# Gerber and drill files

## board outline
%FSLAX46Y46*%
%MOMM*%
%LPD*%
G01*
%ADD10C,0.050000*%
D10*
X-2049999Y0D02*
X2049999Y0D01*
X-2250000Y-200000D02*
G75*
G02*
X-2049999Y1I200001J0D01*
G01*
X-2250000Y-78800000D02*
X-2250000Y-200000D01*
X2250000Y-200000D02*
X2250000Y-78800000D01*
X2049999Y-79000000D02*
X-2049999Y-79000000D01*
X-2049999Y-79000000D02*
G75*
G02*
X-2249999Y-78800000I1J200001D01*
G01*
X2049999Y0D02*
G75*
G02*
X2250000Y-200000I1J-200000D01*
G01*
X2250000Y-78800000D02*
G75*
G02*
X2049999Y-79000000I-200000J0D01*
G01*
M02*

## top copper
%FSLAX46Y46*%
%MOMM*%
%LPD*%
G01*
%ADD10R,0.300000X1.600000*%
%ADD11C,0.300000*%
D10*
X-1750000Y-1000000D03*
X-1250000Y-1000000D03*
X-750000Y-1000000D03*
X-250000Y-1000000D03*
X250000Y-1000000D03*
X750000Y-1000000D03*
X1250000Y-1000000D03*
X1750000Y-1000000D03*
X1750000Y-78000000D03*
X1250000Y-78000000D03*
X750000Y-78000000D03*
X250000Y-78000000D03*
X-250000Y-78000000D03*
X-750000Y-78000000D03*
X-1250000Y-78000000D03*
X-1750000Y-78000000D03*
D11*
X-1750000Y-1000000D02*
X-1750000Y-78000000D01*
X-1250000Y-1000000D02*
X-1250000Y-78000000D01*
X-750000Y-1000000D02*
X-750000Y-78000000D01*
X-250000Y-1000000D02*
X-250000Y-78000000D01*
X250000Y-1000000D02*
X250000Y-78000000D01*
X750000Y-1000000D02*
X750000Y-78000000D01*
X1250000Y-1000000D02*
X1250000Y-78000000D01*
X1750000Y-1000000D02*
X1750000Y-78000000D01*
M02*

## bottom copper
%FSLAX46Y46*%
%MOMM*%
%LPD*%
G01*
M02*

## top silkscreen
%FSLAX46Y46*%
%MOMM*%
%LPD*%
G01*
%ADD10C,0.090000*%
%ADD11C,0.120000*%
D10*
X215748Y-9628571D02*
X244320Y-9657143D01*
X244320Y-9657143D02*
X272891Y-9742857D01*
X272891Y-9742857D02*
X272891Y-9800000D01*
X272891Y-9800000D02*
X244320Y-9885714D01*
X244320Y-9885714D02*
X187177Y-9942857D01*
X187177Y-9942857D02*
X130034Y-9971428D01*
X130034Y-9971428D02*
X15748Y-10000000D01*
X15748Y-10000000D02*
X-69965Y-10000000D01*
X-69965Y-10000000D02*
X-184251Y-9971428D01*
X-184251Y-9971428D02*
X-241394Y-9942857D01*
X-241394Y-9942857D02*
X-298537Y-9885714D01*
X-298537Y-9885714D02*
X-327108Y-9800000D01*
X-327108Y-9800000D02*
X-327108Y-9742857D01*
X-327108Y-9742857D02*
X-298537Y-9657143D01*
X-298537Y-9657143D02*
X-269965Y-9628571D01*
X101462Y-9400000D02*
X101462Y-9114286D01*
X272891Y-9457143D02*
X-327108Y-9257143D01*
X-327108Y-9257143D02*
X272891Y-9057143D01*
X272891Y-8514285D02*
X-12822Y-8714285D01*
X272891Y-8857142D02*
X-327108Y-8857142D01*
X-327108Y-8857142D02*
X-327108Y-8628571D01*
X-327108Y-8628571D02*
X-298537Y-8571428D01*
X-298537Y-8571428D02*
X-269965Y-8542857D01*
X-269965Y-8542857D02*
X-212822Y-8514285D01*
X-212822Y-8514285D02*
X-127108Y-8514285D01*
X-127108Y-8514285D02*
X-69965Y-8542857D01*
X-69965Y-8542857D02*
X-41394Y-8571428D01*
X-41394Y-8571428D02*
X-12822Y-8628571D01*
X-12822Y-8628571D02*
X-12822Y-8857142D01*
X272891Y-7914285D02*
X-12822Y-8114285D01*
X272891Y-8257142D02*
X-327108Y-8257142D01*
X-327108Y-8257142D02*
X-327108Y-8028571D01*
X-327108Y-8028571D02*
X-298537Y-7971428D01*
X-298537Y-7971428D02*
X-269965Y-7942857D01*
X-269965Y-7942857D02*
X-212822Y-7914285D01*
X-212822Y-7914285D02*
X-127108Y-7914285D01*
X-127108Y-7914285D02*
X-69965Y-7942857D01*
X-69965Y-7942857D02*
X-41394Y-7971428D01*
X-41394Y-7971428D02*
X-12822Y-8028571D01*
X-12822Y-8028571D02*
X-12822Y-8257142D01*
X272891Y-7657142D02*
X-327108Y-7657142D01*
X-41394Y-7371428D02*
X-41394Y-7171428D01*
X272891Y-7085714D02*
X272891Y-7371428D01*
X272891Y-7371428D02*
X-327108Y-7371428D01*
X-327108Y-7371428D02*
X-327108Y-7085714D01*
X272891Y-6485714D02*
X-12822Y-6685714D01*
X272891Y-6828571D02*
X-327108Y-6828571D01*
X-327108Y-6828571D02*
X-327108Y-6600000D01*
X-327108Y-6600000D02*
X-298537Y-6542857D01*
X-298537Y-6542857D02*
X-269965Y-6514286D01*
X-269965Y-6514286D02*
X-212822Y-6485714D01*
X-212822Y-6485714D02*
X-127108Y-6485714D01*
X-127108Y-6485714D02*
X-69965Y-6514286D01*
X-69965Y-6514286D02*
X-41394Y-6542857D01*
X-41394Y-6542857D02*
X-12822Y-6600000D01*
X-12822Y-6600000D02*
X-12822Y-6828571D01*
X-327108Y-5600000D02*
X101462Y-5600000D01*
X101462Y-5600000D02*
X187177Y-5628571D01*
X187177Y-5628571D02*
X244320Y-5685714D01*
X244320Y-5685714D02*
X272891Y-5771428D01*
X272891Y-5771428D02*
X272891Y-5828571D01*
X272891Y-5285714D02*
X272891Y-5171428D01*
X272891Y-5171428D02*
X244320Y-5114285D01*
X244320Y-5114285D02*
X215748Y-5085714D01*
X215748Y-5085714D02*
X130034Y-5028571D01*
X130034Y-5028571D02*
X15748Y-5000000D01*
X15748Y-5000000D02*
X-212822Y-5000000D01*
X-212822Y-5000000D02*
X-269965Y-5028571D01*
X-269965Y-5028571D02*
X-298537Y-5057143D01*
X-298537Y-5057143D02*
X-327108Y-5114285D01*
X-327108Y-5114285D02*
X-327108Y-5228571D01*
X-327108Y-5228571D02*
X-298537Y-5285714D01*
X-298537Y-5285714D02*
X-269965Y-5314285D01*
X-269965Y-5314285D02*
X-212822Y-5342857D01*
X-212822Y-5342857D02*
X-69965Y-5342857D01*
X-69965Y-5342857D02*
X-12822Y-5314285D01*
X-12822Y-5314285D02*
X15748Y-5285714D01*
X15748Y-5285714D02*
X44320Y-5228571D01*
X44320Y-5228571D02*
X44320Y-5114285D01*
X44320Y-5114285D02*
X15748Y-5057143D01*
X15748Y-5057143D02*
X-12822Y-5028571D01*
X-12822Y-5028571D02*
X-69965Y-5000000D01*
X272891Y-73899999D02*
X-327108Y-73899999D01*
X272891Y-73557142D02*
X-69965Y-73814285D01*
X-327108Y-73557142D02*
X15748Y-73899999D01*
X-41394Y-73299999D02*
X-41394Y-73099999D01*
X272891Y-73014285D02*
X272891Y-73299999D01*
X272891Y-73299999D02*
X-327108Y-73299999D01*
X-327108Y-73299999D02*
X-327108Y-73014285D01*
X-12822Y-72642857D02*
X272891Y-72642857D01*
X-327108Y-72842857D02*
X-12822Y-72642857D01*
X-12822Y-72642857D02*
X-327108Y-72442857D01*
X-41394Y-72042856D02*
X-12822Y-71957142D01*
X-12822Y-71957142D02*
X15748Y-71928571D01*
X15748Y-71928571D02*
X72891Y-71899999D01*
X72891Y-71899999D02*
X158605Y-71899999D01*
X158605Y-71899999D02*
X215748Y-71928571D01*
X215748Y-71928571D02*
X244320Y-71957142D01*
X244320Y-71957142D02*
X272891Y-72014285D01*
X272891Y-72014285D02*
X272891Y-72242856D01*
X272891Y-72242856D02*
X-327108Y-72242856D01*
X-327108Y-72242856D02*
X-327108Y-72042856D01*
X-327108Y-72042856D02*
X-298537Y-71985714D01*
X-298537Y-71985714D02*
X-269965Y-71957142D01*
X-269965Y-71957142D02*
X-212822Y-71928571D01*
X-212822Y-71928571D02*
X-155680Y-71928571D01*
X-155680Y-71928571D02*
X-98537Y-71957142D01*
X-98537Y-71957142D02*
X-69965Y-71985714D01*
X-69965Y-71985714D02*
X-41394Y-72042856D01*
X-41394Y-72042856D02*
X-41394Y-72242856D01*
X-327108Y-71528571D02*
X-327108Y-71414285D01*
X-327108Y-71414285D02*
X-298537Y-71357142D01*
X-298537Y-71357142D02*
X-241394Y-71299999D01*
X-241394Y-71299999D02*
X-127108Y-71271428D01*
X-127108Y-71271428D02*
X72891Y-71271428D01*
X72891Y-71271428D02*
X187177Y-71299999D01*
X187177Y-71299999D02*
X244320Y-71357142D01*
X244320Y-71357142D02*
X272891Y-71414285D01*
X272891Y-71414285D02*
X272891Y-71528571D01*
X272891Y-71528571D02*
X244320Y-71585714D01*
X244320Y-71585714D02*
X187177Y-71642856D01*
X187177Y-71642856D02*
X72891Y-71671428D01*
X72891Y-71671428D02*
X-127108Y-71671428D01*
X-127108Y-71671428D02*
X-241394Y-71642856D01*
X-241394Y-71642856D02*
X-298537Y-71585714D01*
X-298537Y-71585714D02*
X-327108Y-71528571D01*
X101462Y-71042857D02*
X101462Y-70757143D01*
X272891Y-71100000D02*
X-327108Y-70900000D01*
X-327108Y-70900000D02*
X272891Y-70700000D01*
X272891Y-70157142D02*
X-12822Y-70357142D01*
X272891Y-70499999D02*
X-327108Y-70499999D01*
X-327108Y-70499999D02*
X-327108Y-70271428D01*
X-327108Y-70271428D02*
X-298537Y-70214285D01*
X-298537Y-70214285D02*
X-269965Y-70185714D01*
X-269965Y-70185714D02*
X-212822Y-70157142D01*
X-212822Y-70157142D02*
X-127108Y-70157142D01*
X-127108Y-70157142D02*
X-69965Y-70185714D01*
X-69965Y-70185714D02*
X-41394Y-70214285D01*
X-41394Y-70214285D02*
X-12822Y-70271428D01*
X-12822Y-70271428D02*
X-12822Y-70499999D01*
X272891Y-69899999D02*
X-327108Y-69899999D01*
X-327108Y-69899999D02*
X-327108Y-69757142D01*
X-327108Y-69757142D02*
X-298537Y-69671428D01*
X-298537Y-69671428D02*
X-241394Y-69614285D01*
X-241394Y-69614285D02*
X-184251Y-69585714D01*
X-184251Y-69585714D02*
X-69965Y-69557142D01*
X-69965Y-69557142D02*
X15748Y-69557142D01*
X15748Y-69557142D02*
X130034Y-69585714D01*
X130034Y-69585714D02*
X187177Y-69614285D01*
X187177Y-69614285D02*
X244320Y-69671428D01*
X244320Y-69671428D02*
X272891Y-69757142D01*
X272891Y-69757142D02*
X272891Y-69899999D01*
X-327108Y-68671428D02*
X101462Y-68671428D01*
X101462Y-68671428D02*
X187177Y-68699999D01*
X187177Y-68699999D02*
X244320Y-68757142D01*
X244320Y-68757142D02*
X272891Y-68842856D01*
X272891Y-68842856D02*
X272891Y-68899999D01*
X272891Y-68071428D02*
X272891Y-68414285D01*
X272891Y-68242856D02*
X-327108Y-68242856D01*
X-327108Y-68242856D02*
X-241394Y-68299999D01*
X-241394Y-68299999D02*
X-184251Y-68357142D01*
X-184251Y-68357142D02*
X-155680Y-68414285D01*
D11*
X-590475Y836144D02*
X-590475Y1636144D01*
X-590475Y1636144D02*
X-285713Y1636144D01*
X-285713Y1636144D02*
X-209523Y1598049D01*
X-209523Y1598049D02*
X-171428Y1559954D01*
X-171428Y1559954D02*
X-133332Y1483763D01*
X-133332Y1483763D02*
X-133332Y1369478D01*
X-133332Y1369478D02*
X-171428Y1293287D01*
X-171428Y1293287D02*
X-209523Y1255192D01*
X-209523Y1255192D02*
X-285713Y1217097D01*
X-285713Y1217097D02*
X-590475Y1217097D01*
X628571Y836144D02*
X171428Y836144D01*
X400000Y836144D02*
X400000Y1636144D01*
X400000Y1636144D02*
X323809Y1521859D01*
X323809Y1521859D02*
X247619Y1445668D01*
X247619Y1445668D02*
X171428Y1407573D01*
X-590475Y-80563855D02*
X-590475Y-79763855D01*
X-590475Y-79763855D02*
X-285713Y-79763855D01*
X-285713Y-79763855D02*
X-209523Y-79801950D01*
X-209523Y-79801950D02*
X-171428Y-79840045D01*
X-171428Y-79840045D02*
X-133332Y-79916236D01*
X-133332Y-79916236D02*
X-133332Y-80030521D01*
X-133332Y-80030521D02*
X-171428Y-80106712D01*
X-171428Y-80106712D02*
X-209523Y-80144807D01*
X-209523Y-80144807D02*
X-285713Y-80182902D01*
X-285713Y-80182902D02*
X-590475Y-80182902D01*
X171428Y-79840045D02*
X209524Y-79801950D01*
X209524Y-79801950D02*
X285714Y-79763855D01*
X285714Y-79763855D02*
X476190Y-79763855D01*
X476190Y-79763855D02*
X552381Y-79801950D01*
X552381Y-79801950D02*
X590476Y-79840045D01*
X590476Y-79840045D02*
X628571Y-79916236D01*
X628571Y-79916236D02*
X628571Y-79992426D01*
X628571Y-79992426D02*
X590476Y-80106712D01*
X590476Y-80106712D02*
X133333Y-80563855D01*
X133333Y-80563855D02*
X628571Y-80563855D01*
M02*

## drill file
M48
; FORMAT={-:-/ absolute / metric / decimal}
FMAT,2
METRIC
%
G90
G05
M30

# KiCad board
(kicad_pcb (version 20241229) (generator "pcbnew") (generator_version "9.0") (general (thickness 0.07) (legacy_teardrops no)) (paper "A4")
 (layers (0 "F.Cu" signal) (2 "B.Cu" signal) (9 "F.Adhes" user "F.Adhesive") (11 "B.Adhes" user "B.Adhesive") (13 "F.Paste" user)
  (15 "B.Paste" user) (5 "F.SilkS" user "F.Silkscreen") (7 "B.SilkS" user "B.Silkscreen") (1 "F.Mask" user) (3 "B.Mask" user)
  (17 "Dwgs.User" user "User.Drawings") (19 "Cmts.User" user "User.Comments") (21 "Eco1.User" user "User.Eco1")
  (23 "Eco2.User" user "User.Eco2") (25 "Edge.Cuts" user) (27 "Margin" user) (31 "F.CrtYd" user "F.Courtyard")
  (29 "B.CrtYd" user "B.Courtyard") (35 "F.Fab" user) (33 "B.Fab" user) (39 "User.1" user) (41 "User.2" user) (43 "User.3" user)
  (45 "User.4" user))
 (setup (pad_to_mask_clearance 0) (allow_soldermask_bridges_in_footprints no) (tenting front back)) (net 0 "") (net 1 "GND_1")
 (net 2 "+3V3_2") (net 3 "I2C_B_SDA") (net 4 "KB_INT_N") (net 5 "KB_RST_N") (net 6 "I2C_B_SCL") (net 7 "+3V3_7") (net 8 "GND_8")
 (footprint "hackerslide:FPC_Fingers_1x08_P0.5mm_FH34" (layer "F.Cu") (at 0 0)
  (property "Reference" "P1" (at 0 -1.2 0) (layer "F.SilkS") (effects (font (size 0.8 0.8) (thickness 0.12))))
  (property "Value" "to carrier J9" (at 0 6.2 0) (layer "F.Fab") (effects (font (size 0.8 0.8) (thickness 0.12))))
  (pad "1" smd rect (at -1.75 1) (size 0.3 1.6) (layers "F.Cu" "F.Mask") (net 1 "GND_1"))
  (pad "2" smd rect (at -1.25 1) (size 0.3 1.6) (layers "F.Cu" "F.Mask") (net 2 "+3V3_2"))
  (pad "3" smd rect (at -0.75 1) (size 0.3 1.6) (layers "F.Cu" "F.Mask") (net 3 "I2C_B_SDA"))
  (pad "4" smd rect (at -0.25 1) (size 0.3 1.6) (layers "F.Cu" "F.Mask") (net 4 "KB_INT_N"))
  (pad "5" smd rect (at 0.25 1) (size 0.3 1.6) (layers "F.Cu" "F.Mask") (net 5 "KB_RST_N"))
  (pad "6" smd rect (at 0.75 1) (size 0.3 1.6) (layers "F.Cu" "F.Mask") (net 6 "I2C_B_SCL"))
  (pad "7" smd rect (at 1.25 1) (size 0.3 1.6) (layers "F.Cu" "F.Mask") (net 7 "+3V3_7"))
  (pad "8" smd rect (at 1.75 1) (size 0.3 1.6) (layers "F.Cu" "F.Mask") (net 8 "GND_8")))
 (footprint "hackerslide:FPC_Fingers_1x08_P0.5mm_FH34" (layer "F.Cu") (at 0 79 180)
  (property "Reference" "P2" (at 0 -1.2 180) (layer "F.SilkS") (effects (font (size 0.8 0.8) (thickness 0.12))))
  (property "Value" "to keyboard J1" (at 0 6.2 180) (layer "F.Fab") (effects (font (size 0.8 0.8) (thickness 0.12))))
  (pad "1" smd rect (at -1.75 1 180) (size 0.3 1.6) (layers "F.Cu" "F.Mask") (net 8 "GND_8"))
  (pad "2" smd rect (at -1.25 1 180) (size 0.3 1.6) (layers "F.Cu" "F.Mask") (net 7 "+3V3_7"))
  (pad "3" smd rect (at -0.75 1 180) (size 0.3 1.6) (layers "F.Cu" "F.Mask") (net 6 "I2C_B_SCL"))
  (pad "4" smd rect (at -0.25 1 180) (size 0.3 1.6) (layers "F.Cu" "F.Mask") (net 5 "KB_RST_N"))
  (pad "5" smd rect (at 0.25 1 180) (size 0.3 1.6) (layers "F.Cu" "F.Mask") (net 4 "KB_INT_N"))
  (pad "6" smd rect (at 0.75 1 180) (size 0.3 1.6) (layers "F.Cu" "F.Mask") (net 3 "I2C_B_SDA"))
  (pad "7" smd rect (at 1.25 1 180) (size 0.3 1.6) (layers "F.Cu" "F.Mask") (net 2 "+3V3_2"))
  (pad "8" smd rect (at 1.75 1 180) (size 0.3 1.6) (layers "F.Cu" "F.Mask") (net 1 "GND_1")))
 (gr_line (start -2.049999 0) (end 2.049999 0) (stroke (width 0.05) (type default)) (layer "Edge.Cuts"))
 (gr_arc (start -2.25 0.2) (mid -2.191421 0.058578) (end -2.049999 -0.000001) (stroke (width 0.05) (type default)) (layer "Edge.Cuts"))
 (gr_line (start -2.25 78.8) (end -2.25 0.2) (stroke (width 0.05) (type default)) (layer "Edge.Cuts"))
 (gr_line (start 2.25 0.2) (end 2.25 78.8) (stroke (width 0.05) (type default)) (layer "Edge.Cuts"))
 (gr_line (start 2.049999 79) (end -2.049999 79) (stroke (width 0.05) (type default)) (layer "Edge.Cuts"))
 (gr_arc (start -2.049999 79) (mid -2.19142 78.941421) (end -2.249999 78.8) (stroke (width 0.05) (type default)) (layer "Edge.Cuts"))
 (gr_arc (start 2.049999 0) (mid 2.19142 0.058579) (end 2.249999 0.2) (stroke (width 0.05) (type default)) (layer "Edge.Cuts"))
 (gr_arc (start 2.25 78.8) (mid 2.191421 78.941422) (end 2.049999 79.000001) (stroke (width 0.05) (type default)) (layer "Edge.Cuts"))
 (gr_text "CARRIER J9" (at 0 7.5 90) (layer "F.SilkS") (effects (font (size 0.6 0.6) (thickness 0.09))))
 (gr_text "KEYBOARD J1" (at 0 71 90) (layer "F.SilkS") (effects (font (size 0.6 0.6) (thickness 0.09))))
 (segment (start -1.75 1) (end -1.75 78) (width 0.3) (layer "F.Cu") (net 1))
 (segment (start -1.25 1) (end -1.25 78) (width 0.3) (layer "F.Cu") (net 2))
 (segment (start -0.75 1) (end -0.75 78) (width 0.3) (layer "F.Cu") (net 3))
 (segment (start -0.25 1) (end -0.25 78) (width 0.3) (layer "F.Cu") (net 4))
 (segment (start 0.25 1) (end 0.25 78) (width 0.3) (layer "F.Cu") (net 5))
 (segment (start 0.75 1) (end 0.75 78) (width 0.3) (layer "F.Cu") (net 6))
 (segment (start 1.25 1) (end 1.25 78) (width 0.3) (layer "F.Cu") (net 7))
 (segment (start 1.75 1) (end 1.75 78) (width 0.3) (layer "F.Cu") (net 8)))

